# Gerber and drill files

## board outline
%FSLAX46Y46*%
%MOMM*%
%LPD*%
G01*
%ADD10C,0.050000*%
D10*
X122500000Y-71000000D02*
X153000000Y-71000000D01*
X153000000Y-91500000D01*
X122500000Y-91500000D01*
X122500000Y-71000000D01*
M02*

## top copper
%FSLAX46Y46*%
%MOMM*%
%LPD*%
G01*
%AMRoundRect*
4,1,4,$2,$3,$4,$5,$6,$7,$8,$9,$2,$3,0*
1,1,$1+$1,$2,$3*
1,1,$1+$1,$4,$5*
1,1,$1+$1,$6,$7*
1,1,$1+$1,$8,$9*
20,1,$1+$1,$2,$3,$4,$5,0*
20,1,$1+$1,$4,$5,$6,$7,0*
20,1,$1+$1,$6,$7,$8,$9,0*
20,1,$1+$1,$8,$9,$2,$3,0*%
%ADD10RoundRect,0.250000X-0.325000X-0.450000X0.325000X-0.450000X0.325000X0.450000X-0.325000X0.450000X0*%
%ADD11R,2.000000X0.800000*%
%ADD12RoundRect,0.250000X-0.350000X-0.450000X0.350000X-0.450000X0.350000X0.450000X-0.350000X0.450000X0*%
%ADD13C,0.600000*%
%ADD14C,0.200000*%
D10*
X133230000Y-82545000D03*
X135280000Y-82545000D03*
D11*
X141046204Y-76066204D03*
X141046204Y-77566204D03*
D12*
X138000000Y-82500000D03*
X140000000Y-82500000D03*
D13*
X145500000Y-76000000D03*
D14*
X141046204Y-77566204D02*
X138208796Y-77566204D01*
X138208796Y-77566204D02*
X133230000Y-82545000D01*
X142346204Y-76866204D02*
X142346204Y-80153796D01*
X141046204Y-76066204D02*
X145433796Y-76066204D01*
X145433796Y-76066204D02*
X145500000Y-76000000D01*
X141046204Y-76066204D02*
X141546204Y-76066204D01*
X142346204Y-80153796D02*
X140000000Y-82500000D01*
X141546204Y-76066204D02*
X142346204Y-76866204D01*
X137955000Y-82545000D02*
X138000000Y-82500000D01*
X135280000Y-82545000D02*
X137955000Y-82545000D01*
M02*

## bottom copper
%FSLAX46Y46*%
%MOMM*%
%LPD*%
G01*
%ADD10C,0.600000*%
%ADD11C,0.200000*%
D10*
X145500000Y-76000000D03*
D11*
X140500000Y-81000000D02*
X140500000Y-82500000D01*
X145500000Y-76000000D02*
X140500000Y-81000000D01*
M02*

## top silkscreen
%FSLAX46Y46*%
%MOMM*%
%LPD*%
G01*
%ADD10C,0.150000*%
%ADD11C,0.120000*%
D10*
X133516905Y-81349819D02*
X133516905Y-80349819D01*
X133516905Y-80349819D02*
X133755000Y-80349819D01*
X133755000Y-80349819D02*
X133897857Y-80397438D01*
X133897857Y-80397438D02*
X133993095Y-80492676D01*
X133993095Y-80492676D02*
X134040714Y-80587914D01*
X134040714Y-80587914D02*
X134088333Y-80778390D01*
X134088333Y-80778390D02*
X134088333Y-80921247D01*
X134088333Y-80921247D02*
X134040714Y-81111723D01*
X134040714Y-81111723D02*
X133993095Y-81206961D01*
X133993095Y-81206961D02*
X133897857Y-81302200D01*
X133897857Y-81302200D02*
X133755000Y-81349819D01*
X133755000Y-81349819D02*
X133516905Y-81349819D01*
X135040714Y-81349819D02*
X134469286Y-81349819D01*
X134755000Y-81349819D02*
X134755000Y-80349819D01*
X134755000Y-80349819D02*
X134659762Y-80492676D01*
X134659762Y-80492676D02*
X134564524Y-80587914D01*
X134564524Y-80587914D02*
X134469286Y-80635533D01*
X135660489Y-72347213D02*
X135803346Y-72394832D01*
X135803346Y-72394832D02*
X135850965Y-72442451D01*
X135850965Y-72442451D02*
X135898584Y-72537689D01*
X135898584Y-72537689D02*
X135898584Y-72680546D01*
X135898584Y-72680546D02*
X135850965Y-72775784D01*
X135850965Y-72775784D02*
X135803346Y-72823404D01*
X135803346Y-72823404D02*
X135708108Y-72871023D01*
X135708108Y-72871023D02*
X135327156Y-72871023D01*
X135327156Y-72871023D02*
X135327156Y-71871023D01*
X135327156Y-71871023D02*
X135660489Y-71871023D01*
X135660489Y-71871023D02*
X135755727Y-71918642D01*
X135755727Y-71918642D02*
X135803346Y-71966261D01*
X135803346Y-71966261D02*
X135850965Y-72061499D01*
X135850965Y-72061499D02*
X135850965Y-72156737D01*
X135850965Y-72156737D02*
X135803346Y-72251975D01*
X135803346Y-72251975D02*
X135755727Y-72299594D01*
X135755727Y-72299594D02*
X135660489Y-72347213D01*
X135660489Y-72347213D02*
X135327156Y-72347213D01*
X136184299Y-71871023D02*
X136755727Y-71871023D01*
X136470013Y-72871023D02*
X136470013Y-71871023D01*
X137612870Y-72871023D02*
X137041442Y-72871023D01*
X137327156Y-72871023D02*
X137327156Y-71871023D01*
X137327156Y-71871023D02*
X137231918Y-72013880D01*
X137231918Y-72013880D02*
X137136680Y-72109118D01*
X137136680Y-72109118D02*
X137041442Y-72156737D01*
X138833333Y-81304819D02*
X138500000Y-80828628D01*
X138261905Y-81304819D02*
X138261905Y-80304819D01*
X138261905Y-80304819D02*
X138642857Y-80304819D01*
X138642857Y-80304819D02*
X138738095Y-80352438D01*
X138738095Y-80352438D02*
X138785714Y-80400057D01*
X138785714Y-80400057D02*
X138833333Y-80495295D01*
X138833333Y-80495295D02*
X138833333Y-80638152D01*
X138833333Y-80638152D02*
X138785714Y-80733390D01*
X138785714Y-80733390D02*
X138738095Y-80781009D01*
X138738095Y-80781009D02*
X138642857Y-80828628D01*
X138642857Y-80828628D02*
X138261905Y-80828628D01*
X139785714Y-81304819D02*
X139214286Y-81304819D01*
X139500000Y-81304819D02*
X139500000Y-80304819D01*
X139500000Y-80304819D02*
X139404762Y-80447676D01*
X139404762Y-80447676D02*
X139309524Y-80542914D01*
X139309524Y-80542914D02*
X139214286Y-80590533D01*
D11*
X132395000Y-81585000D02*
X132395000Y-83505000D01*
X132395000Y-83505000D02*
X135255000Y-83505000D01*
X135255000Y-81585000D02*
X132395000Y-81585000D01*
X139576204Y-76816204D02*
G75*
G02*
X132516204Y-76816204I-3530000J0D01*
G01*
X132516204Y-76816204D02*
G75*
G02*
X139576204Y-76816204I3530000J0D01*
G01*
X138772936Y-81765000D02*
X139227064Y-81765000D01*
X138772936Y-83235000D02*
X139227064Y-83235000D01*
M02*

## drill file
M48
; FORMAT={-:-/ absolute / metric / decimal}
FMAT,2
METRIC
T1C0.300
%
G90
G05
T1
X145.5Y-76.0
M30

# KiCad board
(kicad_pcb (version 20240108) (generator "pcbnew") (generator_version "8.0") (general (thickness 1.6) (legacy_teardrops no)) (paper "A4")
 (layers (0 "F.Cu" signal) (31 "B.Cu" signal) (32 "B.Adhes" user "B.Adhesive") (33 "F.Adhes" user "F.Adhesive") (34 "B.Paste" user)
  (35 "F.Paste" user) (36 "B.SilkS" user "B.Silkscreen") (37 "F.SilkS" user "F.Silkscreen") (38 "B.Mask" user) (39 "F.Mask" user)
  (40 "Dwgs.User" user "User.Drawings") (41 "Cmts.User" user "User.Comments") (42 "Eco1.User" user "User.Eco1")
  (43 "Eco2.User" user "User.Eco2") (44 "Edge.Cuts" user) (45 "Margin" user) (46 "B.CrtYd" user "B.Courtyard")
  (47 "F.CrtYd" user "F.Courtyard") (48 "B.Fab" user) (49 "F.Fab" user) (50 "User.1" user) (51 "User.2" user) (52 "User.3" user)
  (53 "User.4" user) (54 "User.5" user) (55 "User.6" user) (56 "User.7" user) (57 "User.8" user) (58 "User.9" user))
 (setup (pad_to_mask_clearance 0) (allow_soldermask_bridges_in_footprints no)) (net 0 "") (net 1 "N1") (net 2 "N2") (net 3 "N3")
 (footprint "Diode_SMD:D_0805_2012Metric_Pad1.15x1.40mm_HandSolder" (layer "F.Cu") (at 134.255 82.545)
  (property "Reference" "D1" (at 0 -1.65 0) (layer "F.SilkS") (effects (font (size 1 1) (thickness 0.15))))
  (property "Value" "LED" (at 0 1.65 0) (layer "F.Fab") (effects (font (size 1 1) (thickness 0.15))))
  (fp_line (start -1.86 -0.96) (end -1.86 0.96) (stroke (width 0.12) (type solid)) (layer "F.SilkS"))
  (fp_line (start -1.86 0.96) (end 1 0.96) (stroke (width 0.12) (type solid)) (layer "F.SilkS"))
  (fp_line (start 1 -0.96) (end -1.86 -0.96) (stroke (width 0.12) (type solid)) (layer "F.SilkS"))
  (pad "1" smd roundrect (at -1.025 0) (size 1.15 1.4) (layers "F.Cu" "F.Paste" "F.Mask") (roundrect_rratio 0.217391) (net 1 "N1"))
  (pad "2" smd roundrect (at 1.025 0) (size 1.15 1.4) (layers "F.Cu" "F.Paste" "F.Mask") (roundrect_rratio 0.217391) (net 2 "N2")))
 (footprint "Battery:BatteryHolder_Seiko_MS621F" (layer "F.Cu") (at 141.046204 76.816204)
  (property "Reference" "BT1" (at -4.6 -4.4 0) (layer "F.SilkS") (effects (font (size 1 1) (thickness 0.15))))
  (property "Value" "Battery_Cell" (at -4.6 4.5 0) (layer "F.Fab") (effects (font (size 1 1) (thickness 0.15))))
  (fp_circle (center -5 0) (end -1.47 0) (stroke (width 0.12) (type solid)) (fill none) (layer "F.SilkS"))
  (pad "1" smd rect (at 0 -0.75) (size 2 0.8) (layers "F.Cu" "F.Paste" "F.Mask") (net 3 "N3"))
  (pad "2" smd rect (at 0 0.75) (size 2 0.8) (layers "F.Cu" "F.Paste" "F.Mask") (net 1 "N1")))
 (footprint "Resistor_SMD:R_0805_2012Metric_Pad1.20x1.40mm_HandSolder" (layer "F.Cu") (at 139 82.5)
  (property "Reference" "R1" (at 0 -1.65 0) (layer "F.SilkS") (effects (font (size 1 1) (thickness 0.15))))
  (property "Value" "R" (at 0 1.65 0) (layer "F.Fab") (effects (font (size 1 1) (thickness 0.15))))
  (fp_line (start -0.227064 -0.735) (end 0.227064 -0.735) (stroke (width 0.12) (type solid)) (layer "F.SilkS"))
  (fp_line (start -0.227064 0.735) (end 0.227064 0.735) (stroke (width 0.12) (type solid)) (layer "F.SilkS"))
  (pad "1" smd roundrect (at -1 0) (size 1.2 1.4) (layers "F.Cu" "F.Paste" "F.Mask") (roundrect_rratio 0.208333) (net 2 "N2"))
  (pad "2" smd roundrect (at 1 0) (size 1.2 1.4) (layers "F.Cu" "F.Paste" "F.Mask") (roundrect_rratio 0.208333) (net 3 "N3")))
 (gr_rect (start 122.5 71) (end 153 91.5) (stroke (width 0.05) (type default)) (fill none) (layer "Edge.Cuts"))
 (segment (start 141.046204 77.566204) (end 138.208796 77.566204) (width 0.2) (layer "F.Cu") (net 1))
 (segment (start 138.208796 77.566204) (end 133.23 82.545) (width 0.2) (layer "F.Cu") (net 1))
 (segment (start 142.346204 76.866204) (end 142.346204 80.153796) (width 0.2) (layer "F.Cu") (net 3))
 (segment (start 141.046204 76.066204) (end 145.433796 76.066204) (width 0.2) (layer "F.Cu") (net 3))
 (segment (start 145.433796 76.066204) (end 145.5 76) (width 0.2) (layer "F.Cu") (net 3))
 (segment (start 141.046204 76.066204) (end 141.546204 76.066204) (width 0.2) (layer "F.Cu") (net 3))
 (segment (start 142.346204 80.153796) (end 140 82.5) (width 0.2) (layer "F.Cu") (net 3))
 (segment (start 141.546204 76.066204) (end 142.346204 76.866204) (width 0.2) (layer "F.Cu") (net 3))
 (via (at 145.5 76) (size 0.6) (drill 0.3) (layers "F.Cu" "B.Cu") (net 3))
 (segment (start 140.5 81) (end 140.5 82.5) (width 0.2) (layer "B.Cu") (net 3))
 (segment (start 145.5 76) (end 140.5 81) (width 0.2) (layer "B.Cu") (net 3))
 (segment (start 137.955 82.545) (end 138 82.5) (width 0.2) (layer "F.Cu") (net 2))
 (segment (start 135.28 82.545) (end 137.955 82.545) (width 0.2) (layer "F.Cu") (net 2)))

